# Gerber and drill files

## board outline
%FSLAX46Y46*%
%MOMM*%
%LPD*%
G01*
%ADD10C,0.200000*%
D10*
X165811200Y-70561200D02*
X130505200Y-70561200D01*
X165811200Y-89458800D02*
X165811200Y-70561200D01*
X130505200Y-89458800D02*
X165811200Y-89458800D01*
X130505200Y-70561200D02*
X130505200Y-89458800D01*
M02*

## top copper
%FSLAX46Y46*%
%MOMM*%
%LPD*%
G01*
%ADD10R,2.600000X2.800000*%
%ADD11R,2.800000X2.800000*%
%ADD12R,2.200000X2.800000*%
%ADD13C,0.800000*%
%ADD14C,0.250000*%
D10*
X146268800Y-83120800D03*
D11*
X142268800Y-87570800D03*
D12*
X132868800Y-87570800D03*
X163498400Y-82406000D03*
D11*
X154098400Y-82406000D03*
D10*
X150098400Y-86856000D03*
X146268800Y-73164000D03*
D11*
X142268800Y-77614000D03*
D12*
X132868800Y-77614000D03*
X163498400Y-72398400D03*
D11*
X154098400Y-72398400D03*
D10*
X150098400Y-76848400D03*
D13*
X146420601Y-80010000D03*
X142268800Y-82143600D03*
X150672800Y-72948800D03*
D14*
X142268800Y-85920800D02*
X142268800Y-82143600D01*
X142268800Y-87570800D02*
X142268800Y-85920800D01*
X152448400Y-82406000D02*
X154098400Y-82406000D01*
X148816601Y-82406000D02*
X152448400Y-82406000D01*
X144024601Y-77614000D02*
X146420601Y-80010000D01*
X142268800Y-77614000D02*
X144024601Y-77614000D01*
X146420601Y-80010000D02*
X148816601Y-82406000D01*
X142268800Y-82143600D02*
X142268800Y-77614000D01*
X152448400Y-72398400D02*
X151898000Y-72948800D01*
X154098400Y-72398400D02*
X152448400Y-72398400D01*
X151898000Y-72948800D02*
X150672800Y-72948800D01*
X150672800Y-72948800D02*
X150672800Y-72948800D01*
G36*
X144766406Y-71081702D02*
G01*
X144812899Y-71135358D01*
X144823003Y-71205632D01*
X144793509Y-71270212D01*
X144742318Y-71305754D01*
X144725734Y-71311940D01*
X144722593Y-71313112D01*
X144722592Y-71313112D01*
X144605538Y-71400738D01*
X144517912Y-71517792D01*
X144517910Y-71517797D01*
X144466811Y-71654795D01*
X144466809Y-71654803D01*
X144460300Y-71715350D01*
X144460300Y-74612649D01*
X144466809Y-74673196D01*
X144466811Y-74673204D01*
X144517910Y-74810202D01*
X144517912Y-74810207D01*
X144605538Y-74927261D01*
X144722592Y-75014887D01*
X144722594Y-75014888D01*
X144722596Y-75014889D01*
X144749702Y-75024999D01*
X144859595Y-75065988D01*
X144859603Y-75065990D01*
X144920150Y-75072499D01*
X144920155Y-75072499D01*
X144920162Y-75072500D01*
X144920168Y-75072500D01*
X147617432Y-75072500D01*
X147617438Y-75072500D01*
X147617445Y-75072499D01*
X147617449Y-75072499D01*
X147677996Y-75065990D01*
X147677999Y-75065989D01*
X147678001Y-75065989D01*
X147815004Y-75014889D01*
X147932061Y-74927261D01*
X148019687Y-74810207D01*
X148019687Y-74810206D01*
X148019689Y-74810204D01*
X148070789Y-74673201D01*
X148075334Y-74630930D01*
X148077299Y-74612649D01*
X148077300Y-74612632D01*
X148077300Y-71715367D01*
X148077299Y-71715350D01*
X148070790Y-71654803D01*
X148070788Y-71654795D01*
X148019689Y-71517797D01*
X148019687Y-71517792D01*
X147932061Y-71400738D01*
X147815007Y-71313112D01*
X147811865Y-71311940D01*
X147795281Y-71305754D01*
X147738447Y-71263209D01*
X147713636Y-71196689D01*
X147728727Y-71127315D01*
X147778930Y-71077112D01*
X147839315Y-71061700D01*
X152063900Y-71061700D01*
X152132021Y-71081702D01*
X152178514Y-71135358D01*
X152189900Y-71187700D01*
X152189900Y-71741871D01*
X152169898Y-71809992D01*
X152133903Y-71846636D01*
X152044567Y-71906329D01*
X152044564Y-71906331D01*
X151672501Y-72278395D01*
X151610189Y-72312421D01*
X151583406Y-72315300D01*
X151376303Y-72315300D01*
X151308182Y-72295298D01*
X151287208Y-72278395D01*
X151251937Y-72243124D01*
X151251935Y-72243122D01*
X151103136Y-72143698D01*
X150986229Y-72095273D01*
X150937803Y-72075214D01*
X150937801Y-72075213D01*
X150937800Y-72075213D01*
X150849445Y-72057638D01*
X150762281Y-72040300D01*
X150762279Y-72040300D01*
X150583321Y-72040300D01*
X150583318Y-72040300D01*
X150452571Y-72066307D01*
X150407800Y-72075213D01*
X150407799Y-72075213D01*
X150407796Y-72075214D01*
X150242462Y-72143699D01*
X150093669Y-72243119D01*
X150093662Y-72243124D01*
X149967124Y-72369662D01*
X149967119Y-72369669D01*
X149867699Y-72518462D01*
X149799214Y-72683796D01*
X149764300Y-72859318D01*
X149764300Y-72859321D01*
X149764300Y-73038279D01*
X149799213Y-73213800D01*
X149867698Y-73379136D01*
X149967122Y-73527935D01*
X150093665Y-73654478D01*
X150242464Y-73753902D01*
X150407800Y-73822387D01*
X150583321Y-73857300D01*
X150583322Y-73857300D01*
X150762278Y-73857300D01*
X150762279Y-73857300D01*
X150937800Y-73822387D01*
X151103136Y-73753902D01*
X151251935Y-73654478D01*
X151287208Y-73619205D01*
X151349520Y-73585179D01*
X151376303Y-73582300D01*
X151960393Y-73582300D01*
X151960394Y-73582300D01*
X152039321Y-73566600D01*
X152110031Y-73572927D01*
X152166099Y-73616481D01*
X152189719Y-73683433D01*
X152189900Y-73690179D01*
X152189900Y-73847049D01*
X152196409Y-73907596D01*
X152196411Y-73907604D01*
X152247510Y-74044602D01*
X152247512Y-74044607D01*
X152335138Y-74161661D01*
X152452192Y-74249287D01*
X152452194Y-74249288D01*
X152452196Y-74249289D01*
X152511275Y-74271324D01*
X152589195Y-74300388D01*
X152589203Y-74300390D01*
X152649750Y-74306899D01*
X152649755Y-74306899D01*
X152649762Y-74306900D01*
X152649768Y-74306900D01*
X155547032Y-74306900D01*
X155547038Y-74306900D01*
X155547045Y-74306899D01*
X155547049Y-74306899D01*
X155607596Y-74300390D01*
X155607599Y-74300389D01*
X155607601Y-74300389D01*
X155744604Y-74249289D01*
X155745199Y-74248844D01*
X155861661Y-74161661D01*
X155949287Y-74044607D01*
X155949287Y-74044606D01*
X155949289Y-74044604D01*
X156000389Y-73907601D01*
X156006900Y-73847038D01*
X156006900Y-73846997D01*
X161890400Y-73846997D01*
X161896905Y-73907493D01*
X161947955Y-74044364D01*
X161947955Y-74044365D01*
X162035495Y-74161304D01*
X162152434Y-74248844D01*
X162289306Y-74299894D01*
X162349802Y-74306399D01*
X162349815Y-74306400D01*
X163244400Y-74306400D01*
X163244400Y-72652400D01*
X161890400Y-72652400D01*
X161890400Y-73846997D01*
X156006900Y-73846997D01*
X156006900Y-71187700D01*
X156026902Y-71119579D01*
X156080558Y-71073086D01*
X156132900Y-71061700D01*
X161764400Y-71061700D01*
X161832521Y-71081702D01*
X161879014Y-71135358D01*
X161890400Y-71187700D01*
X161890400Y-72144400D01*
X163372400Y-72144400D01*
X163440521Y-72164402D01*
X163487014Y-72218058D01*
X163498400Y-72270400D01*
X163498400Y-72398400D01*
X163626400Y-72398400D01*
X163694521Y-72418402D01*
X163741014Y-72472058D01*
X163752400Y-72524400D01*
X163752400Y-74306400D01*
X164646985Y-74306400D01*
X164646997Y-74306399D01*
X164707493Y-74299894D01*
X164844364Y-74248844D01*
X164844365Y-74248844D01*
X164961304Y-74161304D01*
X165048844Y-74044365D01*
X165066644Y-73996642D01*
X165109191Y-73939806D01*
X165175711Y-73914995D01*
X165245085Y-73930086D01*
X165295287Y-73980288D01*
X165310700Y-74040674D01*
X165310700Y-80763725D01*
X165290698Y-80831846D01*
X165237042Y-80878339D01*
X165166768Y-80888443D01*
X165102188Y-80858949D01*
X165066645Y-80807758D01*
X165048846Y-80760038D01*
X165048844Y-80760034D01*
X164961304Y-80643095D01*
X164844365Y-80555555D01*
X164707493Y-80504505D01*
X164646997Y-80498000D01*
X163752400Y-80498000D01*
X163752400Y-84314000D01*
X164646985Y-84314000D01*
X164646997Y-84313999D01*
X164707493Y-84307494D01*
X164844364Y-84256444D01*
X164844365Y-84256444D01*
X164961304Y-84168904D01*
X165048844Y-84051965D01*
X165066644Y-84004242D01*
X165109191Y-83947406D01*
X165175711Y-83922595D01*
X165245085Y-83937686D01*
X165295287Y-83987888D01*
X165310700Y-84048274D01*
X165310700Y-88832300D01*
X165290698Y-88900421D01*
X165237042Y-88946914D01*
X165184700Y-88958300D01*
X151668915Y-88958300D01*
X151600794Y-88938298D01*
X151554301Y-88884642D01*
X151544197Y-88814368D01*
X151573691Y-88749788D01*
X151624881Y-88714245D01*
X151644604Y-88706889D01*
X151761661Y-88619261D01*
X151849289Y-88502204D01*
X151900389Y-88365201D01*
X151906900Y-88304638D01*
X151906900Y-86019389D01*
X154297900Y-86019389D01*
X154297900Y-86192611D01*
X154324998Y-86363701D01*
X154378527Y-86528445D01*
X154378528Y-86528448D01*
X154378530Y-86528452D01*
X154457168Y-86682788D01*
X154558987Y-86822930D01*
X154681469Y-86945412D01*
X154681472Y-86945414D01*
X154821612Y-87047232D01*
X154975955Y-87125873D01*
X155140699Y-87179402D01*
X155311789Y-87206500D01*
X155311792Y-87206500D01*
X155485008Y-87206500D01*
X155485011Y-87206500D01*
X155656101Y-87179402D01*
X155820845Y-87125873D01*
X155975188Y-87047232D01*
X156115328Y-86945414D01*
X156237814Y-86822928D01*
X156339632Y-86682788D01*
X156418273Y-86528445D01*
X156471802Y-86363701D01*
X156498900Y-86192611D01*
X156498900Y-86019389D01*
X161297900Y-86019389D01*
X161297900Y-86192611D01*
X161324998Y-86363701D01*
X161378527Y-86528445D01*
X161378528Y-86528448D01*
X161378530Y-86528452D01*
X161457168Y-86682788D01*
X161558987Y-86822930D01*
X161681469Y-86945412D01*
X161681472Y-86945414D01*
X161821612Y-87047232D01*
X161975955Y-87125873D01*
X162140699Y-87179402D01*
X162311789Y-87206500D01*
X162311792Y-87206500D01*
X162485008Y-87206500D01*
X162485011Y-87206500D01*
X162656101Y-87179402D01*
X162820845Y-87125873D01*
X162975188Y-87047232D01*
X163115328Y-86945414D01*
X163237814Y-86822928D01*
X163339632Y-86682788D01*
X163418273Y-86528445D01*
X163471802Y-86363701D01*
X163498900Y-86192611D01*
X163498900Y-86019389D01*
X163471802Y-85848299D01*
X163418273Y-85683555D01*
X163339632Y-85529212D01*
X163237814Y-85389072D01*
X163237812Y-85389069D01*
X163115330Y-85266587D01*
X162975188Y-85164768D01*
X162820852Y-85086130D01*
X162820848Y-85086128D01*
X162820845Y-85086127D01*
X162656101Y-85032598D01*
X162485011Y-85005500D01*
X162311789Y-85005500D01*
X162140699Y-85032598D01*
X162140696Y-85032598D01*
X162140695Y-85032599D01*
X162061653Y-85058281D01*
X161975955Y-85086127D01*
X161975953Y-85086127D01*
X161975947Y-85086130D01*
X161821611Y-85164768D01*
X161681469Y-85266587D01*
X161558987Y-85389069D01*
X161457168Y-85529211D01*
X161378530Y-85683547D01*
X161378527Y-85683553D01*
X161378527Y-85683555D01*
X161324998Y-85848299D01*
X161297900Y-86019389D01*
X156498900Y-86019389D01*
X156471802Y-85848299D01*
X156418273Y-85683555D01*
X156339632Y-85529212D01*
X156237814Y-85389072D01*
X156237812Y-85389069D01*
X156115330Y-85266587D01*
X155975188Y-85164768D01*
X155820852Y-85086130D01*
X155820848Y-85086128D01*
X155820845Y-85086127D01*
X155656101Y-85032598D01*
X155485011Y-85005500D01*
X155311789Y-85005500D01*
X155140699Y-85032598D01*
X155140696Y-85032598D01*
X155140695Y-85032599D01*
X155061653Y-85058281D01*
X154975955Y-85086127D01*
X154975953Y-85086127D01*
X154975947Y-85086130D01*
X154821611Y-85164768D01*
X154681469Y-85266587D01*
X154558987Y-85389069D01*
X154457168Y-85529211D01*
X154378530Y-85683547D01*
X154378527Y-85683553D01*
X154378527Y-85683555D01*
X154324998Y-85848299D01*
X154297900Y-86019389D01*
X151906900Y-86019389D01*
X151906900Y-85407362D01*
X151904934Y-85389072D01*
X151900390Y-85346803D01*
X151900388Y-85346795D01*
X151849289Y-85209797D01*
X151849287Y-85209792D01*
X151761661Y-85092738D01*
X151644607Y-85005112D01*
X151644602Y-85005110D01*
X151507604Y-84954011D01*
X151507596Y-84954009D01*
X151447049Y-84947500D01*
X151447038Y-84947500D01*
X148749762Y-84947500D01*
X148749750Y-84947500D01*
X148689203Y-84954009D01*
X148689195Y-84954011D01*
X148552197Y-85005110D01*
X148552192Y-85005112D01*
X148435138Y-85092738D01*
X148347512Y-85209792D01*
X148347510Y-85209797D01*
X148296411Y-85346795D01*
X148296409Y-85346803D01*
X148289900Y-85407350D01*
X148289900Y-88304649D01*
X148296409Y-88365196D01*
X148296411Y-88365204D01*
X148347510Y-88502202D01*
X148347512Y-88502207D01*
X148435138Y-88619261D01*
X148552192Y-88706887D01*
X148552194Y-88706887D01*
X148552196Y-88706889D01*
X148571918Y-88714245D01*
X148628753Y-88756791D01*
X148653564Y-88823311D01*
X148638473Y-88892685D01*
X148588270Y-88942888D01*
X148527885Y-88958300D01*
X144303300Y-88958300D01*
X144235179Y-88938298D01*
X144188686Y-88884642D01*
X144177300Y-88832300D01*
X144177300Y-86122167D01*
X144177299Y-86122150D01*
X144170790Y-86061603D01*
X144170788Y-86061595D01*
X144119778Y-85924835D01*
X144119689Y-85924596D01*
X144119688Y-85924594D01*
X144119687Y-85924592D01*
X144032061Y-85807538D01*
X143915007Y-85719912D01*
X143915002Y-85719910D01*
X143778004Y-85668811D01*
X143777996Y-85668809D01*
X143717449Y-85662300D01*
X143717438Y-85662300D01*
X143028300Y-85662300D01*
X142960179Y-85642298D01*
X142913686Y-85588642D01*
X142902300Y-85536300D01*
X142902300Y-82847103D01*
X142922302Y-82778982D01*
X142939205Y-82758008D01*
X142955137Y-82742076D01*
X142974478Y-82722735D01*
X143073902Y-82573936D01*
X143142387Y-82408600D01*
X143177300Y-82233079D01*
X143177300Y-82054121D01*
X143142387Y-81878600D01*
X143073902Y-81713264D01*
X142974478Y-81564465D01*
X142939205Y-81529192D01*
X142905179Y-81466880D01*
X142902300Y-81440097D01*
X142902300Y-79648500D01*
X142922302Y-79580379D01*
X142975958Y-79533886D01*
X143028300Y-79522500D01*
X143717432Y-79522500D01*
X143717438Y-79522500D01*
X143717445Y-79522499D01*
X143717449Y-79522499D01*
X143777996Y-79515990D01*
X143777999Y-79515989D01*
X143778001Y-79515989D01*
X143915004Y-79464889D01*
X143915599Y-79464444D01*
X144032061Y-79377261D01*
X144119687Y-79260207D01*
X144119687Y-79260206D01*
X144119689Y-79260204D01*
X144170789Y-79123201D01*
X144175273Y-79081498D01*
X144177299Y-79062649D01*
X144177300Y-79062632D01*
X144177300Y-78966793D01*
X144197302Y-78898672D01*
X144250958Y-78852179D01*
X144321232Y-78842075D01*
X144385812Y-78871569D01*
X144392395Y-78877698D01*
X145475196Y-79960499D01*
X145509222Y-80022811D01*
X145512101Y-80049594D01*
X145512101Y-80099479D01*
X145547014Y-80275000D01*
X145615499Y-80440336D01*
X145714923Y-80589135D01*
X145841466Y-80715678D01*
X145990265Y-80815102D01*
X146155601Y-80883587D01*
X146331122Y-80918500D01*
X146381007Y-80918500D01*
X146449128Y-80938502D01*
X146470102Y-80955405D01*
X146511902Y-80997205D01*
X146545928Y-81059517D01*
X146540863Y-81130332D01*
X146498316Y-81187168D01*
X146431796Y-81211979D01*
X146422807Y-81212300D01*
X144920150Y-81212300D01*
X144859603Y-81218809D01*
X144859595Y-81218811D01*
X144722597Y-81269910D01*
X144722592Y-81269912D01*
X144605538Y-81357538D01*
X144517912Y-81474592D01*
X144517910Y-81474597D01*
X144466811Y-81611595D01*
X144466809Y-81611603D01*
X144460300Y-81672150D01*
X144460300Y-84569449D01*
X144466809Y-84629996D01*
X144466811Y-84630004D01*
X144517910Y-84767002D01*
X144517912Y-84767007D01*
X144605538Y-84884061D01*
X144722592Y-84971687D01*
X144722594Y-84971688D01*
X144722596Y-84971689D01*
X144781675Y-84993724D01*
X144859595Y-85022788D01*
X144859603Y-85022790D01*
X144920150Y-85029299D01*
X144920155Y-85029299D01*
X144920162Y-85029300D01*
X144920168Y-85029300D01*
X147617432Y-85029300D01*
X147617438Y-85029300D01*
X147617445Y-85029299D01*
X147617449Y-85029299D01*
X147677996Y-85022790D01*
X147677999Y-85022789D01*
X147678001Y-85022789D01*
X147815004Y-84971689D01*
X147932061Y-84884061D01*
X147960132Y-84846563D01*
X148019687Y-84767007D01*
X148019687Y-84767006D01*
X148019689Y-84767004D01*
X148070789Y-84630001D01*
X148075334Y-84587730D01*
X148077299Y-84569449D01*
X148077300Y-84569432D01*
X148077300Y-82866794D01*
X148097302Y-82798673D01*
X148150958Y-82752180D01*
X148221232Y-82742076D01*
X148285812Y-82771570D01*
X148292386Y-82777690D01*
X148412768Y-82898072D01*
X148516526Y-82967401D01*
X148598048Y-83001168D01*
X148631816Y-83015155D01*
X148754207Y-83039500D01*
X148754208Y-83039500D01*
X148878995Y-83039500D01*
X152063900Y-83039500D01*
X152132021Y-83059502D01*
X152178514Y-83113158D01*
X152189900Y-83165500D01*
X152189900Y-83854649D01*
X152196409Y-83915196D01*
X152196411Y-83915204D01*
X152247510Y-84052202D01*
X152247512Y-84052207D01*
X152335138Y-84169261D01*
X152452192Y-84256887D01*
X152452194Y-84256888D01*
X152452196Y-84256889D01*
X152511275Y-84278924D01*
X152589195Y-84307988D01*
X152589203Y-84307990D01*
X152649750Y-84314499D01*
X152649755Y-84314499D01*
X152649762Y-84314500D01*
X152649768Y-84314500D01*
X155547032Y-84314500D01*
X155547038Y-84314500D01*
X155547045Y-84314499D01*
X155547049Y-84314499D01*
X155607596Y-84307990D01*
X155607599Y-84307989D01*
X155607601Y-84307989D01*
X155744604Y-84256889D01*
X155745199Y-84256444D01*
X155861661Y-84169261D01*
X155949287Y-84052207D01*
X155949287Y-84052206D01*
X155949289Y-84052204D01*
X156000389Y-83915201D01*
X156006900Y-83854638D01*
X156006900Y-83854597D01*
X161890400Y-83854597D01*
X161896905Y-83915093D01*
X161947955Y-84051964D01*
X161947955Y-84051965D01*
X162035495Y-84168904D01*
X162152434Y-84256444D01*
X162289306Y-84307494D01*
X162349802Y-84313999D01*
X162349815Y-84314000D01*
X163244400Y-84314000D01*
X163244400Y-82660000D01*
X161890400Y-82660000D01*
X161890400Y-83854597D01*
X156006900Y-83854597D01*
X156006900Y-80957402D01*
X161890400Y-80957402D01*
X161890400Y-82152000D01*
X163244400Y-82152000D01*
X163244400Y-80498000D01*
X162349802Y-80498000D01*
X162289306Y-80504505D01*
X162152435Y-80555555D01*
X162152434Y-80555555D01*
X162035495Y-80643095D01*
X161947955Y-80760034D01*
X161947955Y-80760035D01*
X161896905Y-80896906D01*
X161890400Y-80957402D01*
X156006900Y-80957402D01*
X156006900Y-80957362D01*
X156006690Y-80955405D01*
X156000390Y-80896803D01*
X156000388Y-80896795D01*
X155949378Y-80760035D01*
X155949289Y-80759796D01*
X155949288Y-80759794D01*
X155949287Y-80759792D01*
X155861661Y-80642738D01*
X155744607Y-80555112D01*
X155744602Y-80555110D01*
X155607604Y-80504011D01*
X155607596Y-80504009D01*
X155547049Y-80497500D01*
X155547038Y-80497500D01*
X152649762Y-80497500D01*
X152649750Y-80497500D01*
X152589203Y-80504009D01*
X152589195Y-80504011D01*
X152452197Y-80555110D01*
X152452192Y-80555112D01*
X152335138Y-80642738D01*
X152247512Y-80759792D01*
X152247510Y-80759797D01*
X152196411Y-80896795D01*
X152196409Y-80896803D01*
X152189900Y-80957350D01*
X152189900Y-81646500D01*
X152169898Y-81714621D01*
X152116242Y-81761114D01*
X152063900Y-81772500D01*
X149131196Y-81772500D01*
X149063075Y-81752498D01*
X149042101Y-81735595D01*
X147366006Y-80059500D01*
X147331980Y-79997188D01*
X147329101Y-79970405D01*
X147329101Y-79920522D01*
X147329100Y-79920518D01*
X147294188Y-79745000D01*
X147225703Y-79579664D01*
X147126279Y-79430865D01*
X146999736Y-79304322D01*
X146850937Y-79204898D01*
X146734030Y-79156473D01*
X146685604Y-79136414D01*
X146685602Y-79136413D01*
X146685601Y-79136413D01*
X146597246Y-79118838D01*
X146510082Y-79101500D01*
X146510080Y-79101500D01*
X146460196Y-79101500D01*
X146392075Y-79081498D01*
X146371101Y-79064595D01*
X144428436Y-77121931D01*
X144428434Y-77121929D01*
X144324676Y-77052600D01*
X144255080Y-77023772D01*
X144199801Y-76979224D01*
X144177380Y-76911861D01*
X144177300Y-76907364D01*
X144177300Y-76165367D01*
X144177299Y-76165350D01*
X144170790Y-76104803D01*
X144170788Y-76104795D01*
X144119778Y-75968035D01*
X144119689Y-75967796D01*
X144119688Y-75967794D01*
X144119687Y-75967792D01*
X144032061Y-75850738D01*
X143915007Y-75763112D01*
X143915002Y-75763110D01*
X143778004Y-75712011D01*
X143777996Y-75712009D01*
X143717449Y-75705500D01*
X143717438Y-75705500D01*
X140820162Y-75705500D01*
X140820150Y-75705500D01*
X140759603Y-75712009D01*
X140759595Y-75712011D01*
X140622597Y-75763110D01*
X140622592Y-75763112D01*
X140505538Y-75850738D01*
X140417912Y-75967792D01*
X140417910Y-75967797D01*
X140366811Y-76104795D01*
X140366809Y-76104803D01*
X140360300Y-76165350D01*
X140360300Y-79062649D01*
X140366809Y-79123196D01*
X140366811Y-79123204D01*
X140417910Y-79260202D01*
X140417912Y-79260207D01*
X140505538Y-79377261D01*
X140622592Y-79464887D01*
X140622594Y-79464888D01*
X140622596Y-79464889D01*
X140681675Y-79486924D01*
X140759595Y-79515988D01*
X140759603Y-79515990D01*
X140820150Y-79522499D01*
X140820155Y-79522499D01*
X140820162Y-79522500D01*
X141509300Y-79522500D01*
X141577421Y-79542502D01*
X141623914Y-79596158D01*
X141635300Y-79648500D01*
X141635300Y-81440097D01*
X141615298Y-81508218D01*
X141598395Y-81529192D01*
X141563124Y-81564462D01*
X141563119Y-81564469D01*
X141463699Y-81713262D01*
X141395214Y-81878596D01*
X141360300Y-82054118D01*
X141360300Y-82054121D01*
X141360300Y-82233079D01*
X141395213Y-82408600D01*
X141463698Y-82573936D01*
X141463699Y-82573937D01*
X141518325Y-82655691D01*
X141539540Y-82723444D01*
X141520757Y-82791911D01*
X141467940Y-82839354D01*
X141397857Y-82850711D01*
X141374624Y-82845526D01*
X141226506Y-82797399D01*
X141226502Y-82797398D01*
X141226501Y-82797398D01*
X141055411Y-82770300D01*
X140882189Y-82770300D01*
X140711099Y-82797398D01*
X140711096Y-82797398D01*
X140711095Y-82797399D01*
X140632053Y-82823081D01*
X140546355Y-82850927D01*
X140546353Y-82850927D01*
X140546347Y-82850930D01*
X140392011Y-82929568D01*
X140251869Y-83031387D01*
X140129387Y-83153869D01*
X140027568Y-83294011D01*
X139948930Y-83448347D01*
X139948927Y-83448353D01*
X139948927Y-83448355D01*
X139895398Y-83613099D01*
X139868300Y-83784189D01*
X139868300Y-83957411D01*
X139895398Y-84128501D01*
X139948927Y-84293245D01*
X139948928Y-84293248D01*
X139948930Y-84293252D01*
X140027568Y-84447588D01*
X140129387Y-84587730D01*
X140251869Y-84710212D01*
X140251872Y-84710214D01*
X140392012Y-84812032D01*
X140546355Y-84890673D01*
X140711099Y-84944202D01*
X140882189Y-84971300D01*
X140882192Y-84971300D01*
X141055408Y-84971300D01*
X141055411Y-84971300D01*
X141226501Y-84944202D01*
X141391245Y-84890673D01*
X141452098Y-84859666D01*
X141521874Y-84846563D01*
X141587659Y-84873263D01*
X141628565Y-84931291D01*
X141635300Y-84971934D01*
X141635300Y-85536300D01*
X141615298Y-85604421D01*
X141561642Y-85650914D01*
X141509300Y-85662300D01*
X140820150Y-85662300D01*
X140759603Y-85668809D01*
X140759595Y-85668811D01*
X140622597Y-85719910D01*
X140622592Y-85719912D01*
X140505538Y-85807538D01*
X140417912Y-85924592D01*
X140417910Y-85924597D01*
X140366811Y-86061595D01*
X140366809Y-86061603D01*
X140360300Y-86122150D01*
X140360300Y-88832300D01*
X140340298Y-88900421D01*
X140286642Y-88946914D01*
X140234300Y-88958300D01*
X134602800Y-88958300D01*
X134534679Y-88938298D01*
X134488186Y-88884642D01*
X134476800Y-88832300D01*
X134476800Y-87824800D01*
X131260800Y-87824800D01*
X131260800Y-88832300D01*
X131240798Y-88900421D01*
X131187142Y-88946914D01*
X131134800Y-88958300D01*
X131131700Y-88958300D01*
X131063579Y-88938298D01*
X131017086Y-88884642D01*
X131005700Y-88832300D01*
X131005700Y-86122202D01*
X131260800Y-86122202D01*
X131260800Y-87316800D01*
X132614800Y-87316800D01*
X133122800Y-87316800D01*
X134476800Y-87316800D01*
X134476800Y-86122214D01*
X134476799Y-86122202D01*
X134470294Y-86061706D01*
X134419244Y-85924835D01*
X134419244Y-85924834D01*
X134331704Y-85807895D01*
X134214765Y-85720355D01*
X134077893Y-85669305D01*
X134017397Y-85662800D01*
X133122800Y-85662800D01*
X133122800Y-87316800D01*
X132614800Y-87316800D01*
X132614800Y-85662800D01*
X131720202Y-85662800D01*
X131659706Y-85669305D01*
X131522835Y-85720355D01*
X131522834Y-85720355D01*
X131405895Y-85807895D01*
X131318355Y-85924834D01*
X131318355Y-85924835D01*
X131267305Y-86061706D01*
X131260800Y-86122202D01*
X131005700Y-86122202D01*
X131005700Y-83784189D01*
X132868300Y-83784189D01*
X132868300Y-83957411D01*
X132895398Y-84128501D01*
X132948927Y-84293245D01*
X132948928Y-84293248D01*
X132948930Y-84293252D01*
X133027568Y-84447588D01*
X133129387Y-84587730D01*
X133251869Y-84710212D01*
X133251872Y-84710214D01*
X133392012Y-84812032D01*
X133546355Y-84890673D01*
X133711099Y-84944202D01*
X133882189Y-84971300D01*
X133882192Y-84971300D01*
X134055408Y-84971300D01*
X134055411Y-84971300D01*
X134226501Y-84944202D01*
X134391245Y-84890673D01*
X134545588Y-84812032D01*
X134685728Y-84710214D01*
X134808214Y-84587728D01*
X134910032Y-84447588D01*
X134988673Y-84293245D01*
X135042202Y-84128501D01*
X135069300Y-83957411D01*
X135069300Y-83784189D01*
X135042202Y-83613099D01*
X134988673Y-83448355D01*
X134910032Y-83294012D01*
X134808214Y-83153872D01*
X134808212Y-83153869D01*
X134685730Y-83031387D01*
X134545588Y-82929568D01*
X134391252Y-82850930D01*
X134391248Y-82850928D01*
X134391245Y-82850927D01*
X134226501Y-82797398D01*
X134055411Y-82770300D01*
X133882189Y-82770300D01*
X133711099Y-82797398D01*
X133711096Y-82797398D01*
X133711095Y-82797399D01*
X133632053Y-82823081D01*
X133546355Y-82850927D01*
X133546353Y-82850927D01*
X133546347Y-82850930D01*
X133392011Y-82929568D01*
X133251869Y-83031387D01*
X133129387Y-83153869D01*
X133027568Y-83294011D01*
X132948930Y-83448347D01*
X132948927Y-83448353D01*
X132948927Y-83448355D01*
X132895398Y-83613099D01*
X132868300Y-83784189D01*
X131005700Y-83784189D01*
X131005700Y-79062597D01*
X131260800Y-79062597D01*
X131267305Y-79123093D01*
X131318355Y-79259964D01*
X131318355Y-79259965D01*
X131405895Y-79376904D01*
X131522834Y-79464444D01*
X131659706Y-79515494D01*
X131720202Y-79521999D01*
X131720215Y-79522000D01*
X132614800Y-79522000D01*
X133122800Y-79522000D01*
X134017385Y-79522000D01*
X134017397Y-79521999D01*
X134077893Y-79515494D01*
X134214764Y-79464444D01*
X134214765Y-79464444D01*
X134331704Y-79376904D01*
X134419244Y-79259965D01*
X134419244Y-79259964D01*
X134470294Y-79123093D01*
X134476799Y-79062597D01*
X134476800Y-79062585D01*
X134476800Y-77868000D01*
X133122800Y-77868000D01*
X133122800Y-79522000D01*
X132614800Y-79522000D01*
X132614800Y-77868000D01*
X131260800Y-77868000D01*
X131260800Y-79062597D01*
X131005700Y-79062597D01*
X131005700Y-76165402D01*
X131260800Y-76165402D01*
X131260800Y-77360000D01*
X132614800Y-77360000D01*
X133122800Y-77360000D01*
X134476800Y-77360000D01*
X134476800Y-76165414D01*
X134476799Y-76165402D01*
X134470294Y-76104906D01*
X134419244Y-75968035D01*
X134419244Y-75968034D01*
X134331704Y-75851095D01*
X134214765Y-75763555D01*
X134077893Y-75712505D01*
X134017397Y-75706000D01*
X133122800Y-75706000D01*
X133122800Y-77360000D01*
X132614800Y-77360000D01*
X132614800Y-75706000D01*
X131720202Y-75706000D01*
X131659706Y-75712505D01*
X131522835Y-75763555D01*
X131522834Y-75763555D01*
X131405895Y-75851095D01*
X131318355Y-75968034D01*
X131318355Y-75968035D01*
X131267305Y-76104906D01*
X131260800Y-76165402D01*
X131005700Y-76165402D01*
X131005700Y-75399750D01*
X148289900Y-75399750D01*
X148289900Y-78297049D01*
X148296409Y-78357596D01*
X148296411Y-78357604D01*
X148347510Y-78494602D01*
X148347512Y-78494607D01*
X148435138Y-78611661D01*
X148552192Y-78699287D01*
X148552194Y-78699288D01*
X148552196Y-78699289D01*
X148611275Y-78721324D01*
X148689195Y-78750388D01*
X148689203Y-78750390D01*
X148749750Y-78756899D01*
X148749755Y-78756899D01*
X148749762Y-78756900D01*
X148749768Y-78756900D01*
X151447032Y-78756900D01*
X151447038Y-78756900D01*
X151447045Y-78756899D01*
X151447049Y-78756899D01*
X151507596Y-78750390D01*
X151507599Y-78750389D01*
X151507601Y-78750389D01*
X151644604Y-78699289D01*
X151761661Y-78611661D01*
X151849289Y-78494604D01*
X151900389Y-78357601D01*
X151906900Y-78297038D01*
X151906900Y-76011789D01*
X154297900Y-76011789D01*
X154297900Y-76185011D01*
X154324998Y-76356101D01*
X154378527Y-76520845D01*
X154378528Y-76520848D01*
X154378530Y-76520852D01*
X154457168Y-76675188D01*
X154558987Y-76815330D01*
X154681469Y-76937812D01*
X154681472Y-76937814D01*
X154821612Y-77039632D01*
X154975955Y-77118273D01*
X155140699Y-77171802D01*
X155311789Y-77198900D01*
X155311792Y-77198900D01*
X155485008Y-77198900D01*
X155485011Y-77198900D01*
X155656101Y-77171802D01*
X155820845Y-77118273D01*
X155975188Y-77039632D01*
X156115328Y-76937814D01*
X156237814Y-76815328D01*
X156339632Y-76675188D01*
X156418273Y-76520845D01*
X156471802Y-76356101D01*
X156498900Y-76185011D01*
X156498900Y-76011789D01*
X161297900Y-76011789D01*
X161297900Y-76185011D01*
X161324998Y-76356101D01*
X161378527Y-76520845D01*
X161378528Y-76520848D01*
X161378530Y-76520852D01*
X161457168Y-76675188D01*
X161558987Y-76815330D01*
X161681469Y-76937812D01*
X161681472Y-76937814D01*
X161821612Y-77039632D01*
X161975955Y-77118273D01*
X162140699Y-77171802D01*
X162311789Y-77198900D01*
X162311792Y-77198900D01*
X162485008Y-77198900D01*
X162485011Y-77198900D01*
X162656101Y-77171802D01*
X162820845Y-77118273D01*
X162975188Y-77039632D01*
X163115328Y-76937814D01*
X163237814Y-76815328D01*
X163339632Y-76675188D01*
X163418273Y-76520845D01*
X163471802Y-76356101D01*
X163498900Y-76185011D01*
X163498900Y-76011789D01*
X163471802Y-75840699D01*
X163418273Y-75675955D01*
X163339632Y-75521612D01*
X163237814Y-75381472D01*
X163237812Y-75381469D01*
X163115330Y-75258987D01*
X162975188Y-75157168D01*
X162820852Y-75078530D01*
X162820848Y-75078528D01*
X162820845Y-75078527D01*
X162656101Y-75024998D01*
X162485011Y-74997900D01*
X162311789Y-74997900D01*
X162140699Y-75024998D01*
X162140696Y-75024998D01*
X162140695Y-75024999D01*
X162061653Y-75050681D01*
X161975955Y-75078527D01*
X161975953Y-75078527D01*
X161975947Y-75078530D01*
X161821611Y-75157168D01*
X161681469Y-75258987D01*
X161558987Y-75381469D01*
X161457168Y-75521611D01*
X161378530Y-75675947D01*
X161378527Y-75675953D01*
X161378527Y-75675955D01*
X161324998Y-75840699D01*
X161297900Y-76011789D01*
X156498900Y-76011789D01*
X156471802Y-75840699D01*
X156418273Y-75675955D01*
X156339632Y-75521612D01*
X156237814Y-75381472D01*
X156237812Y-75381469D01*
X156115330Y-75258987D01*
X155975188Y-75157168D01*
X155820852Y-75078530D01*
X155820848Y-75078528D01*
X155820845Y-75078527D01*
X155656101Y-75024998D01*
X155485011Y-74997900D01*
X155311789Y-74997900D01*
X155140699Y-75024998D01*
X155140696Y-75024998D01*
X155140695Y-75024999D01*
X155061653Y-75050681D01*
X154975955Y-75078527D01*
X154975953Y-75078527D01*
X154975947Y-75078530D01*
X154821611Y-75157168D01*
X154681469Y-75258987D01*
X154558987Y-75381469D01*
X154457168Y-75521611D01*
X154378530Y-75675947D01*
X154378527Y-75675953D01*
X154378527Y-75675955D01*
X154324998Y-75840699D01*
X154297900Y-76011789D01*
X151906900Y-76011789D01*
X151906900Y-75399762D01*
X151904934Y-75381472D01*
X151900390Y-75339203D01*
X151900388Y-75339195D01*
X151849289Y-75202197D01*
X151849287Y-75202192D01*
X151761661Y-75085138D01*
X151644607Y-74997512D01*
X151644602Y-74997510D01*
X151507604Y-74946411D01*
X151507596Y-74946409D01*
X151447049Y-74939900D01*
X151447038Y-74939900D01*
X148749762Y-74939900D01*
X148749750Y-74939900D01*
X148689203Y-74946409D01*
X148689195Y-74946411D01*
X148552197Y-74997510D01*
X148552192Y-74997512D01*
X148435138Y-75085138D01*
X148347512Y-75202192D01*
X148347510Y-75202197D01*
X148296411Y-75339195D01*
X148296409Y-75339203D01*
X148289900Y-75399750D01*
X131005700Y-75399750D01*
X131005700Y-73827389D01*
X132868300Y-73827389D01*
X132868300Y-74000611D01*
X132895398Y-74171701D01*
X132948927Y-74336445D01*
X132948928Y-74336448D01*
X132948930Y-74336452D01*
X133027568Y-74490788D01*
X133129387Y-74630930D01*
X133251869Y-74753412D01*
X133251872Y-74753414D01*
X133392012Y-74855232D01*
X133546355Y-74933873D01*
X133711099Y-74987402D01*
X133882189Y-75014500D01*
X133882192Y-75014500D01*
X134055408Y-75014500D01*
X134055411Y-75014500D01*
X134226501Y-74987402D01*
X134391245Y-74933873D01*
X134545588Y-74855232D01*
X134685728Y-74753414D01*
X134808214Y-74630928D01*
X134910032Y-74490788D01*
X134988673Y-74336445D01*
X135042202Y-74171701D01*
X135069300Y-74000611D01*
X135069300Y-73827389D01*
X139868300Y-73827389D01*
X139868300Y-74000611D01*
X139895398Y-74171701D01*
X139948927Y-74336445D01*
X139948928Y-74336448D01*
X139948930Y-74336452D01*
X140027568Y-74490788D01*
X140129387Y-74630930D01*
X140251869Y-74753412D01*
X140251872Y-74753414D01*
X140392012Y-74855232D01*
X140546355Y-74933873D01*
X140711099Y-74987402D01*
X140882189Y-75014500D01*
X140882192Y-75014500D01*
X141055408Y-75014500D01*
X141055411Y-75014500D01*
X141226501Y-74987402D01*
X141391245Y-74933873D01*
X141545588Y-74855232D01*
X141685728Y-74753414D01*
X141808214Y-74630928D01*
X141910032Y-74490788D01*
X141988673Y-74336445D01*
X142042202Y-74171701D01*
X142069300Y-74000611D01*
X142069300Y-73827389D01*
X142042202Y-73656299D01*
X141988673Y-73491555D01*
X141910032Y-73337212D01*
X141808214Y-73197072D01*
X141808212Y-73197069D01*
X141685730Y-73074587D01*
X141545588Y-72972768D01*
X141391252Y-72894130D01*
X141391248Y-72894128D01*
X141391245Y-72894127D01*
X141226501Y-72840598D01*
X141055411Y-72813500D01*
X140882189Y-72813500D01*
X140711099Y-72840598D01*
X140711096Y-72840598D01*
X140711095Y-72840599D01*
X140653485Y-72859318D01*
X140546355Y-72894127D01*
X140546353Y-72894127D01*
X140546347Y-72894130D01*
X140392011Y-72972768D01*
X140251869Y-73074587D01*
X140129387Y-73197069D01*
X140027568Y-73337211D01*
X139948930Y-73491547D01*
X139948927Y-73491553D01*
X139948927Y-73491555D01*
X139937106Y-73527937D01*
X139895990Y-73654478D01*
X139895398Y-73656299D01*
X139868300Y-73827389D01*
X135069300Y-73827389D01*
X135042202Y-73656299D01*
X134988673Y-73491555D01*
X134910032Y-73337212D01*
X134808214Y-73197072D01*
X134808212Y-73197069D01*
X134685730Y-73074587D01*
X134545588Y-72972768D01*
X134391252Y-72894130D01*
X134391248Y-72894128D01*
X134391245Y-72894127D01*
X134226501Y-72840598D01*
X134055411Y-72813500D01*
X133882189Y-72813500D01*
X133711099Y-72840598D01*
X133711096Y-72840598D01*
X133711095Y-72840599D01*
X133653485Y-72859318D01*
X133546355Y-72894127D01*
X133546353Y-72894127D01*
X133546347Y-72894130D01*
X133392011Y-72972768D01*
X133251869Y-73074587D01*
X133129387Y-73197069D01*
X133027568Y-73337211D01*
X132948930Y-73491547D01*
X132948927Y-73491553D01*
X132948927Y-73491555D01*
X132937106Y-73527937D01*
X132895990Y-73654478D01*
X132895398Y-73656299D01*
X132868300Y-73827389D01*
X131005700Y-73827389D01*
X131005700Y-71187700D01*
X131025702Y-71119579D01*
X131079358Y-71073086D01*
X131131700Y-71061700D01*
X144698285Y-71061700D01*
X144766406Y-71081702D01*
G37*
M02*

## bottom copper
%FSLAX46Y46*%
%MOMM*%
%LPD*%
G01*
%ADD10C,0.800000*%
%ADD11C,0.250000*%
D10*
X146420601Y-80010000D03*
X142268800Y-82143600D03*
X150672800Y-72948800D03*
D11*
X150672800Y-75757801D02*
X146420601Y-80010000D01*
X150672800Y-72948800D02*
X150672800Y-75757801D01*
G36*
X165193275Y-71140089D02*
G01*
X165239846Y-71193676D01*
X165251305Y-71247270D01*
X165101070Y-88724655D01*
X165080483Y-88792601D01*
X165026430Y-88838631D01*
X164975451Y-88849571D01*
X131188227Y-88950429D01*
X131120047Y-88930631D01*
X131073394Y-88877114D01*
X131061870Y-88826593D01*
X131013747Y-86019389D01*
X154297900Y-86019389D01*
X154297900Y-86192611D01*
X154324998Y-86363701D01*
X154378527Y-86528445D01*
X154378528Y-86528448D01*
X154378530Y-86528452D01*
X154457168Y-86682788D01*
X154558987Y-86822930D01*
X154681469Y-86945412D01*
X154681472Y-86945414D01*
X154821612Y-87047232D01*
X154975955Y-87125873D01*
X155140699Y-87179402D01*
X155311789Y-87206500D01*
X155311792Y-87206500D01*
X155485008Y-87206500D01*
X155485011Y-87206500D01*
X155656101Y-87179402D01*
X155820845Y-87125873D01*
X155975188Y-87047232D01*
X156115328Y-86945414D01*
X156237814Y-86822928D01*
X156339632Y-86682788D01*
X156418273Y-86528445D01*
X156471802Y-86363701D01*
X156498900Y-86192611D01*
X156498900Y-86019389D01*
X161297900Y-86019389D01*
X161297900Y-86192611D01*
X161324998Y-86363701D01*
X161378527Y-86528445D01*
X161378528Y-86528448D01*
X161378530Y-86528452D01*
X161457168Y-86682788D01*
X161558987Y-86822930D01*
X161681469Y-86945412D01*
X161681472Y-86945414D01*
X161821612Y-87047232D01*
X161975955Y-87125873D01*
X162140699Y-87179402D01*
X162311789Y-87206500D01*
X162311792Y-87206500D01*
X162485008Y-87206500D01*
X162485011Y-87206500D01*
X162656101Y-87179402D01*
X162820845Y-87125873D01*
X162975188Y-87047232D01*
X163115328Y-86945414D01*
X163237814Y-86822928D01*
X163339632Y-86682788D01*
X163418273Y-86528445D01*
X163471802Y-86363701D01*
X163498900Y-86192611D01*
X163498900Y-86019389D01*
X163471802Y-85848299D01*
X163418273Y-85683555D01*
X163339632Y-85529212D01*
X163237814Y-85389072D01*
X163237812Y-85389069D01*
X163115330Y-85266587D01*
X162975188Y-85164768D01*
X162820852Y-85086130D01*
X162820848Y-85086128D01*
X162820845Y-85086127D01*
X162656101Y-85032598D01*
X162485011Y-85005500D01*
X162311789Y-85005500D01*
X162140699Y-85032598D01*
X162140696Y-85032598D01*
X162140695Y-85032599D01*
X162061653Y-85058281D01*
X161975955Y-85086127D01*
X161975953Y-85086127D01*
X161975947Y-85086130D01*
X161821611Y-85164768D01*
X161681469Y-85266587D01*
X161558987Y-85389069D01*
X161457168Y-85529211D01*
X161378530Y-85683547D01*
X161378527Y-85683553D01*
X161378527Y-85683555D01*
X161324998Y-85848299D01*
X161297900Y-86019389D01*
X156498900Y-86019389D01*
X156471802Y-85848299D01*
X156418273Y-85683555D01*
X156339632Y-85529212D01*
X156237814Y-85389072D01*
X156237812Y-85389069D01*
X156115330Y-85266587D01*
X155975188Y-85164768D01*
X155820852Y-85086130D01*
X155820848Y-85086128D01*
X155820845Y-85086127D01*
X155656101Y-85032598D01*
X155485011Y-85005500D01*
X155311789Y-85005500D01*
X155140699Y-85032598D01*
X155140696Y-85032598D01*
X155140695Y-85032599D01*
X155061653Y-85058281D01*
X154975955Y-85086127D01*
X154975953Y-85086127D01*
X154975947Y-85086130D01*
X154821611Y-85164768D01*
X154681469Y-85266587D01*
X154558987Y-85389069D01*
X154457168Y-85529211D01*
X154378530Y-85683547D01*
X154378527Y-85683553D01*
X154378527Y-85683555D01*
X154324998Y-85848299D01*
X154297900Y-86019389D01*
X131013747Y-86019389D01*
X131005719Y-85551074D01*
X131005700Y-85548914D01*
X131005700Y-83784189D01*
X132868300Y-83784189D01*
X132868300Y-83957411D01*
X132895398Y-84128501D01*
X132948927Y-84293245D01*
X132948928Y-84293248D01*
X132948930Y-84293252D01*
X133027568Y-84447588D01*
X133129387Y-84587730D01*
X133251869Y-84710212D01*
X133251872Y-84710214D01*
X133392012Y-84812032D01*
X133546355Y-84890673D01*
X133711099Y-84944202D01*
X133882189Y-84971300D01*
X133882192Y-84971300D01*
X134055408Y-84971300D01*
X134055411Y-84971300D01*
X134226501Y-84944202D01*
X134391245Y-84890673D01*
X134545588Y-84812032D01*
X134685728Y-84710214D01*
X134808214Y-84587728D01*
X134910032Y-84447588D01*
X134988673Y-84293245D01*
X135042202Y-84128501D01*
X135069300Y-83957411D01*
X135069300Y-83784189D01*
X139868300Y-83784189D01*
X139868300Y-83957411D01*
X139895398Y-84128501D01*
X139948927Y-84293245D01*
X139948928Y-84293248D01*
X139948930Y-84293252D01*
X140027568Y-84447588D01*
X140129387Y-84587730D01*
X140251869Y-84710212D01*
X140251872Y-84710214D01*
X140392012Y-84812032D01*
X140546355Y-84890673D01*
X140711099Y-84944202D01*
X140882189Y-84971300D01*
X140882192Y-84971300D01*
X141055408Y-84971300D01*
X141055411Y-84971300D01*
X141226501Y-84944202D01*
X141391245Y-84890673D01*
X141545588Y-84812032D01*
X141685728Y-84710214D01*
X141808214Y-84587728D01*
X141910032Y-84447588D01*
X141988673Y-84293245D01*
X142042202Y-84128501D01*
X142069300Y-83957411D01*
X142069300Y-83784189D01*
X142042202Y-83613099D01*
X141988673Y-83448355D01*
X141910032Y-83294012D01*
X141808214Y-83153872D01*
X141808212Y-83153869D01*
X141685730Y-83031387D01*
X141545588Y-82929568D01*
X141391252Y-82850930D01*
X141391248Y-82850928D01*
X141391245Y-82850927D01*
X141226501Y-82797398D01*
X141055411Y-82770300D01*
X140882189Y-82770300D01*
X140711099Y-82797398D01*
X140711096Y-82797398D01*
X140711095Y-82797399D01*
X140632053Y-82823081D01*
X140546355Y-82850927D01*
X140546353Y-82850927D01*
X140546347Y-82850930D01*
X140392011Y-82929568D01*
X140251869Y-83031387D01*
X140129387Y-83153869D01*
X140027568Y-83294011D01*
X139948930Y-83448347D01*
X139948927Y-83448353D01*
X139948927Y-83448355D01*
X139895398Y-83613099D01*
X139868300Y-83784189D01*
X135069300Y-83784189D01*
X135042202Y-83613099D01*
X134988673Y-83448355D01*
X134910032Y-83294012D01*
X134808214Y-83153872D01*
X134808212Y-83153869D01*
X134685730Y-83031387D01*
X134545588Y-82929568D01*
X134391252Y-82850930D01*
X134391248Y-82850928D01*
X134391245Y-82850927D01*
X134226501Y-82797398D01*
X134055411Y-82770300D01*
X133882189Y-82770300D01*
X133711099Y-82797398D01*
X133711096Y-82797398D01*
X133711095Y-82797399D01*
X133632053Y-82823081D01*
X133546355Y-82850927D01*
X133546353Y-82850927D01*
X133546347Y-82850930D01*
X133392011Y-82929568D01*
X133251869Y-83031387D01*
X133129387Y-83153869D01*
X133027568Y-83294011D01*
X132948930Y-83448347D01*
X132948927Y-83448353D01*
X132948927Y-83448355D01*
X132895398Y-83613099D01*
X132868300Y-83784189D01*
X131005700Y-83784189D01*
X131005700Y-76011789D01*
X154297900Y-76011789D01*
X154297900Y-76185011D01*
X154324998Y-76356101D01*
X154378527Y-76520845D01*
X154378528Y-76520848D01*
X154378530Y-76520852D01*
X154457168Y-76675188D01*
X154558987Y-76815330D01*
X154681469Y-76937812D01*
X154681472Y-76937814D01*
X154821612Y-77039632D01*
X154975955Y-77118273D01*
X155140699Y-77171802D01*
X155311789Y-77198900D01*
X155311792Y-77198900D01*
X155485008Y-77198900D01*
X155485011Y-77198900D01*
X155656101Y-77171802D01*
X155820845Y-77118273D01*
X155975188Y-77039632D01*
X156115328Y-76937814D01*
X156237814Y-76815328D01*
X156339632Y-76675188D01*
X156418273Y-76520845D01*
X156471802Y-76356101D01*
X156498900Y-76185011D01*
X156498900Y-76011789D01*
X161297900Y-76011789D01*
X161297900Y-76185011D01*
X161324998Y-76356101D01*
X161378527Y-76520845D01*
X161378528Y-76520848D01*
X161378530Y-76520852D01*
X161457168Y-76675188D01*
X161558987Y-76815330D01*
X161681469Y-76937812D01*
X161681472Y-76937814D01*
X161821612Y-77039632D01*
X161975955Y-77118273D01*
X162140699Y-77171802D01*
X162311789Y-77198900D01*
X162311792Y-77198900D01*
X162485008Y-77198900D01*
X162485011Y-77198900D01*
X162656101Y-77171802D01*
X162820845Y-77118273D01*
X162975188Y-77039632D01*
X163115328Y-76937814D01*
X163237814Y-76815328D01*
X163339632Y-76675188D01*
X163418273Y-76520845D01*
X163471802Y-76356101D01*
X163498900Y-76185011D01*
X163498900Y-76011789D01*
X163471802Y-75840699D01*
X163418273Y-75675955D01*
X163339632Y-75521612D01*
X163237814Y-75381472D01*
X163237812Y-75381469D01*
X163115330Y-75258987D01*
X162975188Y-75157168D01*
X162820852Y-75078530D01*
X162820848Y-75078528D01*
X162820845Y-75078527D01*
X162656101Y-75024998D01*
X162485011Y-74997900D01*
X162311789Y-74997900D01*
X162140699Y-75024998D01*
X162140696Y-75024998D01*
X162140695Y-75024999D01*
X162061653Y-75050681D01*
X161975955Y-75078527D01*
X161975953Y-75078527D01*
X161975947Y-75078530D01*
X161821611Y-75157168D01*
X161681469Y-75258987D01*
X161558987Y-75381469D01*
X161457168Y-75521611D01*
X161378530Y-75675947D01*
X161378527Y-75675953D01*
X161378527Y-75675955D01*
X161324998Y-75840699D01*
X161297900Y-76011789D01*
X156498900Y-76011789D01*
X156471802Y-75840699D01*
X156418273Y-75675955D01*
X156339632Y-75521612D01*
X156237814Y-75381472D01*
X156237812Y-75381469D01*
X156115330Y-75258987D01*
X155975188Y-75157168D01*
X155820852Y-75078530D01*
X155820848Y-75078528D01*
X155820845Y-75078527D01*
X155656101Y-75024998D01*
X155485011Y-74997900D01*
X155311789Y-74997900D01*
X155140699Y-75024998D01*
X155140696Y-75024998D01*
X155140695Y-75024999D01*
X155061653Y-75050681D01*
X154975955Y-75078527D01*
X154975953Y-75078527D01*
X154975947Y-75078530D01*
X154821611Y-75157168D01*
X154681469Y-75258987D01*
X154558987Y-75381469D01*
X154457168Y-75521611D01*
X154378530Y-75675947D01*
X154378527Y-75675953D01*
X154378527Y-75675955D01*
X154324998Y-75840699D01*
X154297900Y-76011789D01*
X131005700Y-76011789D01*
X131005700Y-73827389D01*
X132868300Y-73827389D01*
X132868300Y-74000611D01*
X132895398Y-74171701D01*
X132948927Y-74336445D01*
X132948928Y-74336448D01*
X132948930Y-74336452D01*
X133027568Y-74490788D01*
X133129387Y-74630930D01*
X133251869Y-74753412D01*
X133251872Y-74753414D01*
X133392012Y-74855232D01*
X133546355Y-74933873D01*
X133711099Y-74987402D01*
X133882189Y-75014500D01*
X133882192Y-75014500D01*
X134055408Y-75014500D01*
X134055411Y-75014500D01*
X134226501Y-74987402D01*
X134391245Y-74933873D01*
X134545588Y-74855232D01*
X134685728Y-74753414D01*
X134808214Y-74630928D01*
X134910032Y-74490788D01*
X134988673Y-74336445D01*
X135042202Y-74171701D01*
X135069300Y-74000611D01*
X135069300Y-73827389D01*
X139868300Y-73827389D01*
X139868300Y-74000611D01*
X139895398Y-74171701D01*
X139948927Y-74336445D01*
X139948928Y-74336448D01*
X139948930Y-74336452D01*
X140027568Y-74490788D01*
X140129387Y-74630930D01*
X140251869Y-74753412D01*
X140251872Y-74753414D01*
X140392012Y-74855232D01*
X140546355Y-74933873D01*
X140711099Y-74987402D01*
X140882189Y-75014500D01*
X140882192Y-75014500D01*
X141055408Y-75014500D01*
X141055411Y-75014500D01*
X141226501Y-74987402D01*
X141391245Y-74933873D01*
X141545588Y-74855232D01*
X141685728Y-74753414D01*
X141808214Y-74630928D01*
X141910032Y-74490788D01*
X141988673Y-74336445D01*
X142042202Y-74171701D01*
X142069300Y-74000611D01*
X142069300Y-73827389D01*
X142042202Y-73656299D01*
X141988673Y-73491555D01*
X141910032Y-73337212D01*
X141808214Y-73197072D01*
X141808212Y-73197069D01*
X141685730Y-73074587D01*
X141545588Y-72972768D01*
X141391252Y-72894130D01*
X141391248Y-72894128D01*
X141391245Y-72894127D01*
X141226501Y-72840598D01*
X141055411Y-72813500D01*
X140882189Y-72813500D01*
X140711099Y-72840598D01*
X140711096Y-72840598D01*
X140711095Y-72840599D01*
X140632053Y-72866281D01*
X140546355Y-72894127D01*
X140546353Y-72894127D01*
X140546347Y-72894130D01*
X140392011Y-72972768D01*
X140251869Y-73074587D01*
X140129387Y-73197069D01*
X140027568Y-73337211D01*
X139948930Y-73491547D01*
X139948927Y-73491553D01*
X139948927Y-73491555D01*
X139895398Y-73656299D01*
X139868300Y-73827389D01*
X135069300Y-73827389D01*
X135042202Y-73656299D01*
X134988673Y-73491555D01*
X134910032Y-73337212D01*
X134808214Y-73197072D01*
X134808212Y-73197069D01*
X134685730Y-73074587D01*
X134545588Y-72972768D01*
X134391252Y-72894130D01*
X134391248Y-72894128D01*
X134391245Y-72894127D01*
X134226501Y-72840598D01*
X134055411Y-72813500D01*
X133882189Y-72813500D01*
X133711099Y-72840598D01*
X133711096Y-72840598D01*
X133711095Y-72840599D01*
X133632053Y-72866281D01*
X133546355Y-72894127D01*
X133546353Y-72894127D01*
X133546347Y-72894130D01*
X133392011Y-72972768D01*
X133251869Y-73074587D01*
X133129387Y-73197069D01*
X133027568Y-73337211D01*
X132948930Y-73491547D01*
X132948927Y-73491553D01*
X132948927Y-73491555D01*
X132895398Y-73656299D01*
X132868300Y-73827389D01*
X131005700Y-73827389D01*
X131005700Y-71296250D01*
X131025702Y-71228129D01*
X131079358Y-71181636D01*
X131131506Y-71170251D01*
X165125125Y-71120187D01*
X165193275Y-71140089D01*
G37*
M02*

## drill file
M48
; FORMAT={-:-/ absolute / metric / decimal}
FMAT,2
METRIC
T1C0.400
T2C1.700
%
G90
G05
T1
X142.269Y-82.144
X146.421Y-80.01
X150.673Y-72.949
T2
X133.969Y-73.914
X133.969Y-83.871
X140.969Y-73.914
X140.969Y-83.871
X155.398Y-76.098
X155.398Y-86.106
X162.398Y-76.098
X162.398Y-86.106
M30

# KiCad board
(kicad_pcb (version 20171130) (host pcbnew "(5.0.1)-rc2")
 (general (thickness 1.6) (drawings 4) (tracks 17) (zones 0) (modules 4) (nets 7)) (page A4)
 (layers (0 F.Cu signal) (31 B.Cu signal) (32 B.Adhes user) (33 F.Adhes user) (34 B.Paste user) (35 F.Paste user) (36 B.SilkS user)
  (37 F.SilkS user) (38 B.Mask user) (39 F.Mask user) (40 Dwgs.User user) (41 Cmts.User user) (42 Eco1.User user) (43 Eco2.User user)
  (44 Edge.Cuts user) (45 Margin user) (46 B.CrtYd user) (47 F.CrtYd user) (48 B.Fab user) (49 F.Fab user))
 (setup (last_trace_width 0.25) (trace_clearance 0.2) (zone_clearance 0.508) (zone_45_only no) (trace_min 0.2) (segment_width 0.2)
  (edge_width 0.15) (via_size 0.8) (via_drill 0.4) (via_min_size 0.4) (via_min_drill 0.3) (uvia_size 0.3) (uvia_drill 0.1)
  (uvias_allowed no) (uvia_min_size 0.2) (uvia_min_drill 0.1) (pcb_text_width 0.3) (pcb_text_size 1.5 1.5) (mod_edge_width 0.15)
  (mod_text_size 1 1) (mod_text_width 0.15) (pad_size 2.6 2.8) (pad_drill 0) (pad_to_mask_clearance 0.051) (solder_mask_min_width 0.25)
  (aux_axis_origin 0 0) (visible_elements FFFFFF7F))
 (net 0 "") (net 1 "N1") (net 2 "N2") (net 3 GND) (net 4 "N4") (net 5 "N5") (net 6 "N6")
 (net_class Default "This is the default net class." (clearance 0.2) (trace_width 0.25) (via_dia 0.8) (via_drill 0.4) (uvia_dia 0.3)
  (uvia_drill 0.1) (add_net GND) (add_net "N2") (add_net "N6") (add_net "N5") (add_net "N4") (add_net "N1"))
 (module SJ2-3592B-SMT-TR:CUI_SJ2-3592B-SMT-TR (layer F.Cu) (at 137.7188 83.8708)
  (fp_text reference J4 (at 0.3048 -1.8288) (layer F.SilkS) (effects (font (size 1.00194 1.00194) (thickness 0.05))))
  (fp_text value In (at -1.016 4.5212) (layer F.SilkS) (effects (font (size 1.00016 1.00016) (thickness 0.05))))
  (pad Hole np_thru_hole circle (at 3.25 0) (size 1.7 1.7) (drill 1.7) (layers *.Cu *.Mask F.SilkS))
  (pad Hole np_thru_hole circle (at -3.75 0) (size 1.7 1.7) (drill 1.7) (layers *.Cu *.Mask F.SilkS))
  (pad TN smd rect (at 8.55 -0.75) (size 2.6 2.8) (layers F.Cu F.Paste F.Mask) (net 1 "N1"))
  (pad T smd rect (at 4.55 3.7) (size 2.8 2.8) (layers F.Cu F.Paste F.Mask) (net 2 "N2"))
  (pad S smd rect (at -4.85 3.7) (size 2.2 2.8) (layers F.Cu F.Paste F.Mask) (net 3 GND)))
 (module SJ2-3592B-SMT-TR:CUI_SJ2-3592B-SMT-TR (layer F.Cu) (at 158.6484 86.106 180)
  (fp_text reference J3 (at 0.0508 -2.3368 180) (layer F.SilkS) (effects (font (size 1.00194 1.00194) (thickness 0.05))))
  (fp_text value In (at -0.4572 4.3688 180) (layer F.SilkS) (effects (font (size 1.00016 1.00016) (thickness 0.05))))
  (pad S smd rect (at -4.85 3.7 180) (size 2.2 2.8) (layers F.Cu F.Paste F.Mask) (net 3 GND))
  (pad T smd rect (at 4.55 3.7 180) (size 2.8 2.8) (layers F.Cu F.Paste F.Mask) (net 2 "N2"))
  (pad TN smd rect (at 8.55 -0.75 180) (size 2.6 2.8) (layers F.Cu F.Paste F.Mask) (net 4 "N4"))
  (pad Hole np_thru_hole circle (at -3.75 0 180) (size 1.7 1.7) (drill 1.7) (layers *.Cu *.Mask F.SilkS))
  (pad Hole np_thru_hole circle (at 3.25 0 180) (size 1.7 1.7) (drill 1.7) (layers *.Cu *.Mask F.SilkS)))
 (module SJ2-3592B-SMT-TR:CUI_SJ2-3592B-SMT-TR (layer F.Cu) (at 137.7188 73.914)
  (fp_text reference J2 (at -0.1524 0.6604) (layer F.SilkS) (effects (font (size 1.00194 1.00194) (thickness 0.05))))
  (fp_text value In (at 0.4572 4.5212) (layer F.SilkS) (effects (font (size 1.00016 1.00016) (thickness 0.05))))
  (pad Hole np_thru_hole circle (at 3.25 0) (size 1.7 1.7) (drill 1.7) (layers *.Cu *.Mask F.SilkS))
  (pad Hole np_thru_hole circle (at -3.75 0) (size 1.7 1.7) (drill 1.7) (layers *.Cu *.Mask F.SilkS))
  (pad TN smd rect (at 8.55 -0.75) (size 2.6 2.8) (layers F.Cu F.Paste F.Mask) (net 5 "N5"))
  (pad T smd rect (at 4.55 3.7) (size 2.8 2.8) (layers F.Cu F.Paste F.Mask) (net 2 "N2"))
  (pad S smd rect (at -4.85 3.7) (size 2.2 2.8) (layers F.Cu F.Paste F.Mask) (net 3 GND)))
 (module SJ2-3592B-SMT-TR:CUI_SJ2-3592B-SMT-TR (layer F.Cu) (at 158.6484 76.0984 180)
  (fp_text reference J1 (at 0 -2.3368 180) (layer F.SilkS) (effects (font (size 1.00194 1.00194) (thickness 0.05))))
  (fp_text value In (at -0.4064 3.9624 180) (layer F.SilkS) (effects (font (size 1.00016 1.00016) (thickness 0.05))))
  (pad S smd rect (at -4.85 3.7 180) (size 2.2 2.8) (layers F.Cu F.Paste F.Mask) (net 3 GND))
  (pad T smd rect (at 4.55 3.7 180) (size 2.8 2.8) (layers F.Cu F.Paste F.Mask) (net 2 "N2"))
  (pad TN smd rect (at 8.55 -0.75 180) (size 2.6 2.8) (layers F.Cu F.Paste F.Mask) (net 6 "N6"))
  (pad Hole np_thru_hole circle (at -3.75 0 180) (size 1.7 1.7) (drill 1.7) (layers *.Cu *.Mask F.SilkS))
  (pad Hole np_thru_hole circle (at 3.25 0 180) (size 1.7 1.7) (drill 1.7) (layers *.Cu *.Mask F.SilkS)))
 (gr_line (start 165.8112 70.5612) (end 130.5052 70.5612) (layer Edge.Cuts) (width 0.2))
 (gr_line (start 165.8112 89.4588) (end 165.8112 70.5612) (layer Edge.Cuts) (width 0.2))
 (gr_line (start 130.5052 89.4588) (end 165.8112 89.4588) (layer Edge.Cuts) (width 0.2))
 (gr_line (start 130.5052 70.5612) (end 130.5052 89.4588) (layer Edge.Cuts) (width 0.2))
 (segment (start 142.2688 85.9208) (end 142.2688 82.1436) (width 0.25) (layer F.Cu) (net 2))
 (segment (start 142.2688 87.5708) (end 142.2688 85.9208) (width 0.25) (layer F.Cu) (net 2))
 (segment (start 152.4484 82.406) (end 154.0984 82.406) (width 0.25) (layer F.Cu) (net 2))
 (segment (start 148.816601 82.406) (end 152.4484 82.406) (width 0.25) (layer F.Cu) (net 2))
 (segment (start 144.024601 77.614) (end 146.420601 80.01) (width 0.25) (layer F.Cu) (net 2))
 (segment (start 142.2688 77.614) (end 144.024601 77.614) (width 0.25) (layer F.Cu) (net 2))
 (segment (start 146.420601 80.01) (end 148.816601 82.406) (width 0.25) (layer F.Cu) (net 2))
 (via (at 146.420601 80.01) (size 0.8) (drill 0.4) (layers F.Cu B.Cu) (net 2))
 (segment (start 142.2688 82.1436) (end 142.2688 77.614) (width 0.25) (layer F.Cu) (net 2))
 (via (at 142.2688 82.1436) (size 0.8) (drill 0.4) (layers F.Cu B.Cu) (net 2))
 (segment (start 152.4484 72.3984) (end 151.898 72.9488) (width 0.25) (layer F.Cu) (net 2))
 (segment (start 154.0984 72.3984) (end 152.4484 72.3984) (width 0.25) (layer F.Cu) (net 2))
 (segment (start 151.898 72.9488) (end 150.6728 72.9488) (width 0.25) (layer F.Cu) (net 2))
 (segment (start 150.6728 72.9488) (end 150.6728 72.9488) (width 0.25) (layer F.Cu) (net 2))
 (via (at 150.6728 72.9488) (size 0.8) (drill 0.4) (layers F.Cu B.Cu) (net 2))
 (segment (start 150.6728 75.757801) (end 146.420601 80.01) (width 0.25) (layer B.Cu) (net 2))
 (segment (start 150.6728 72.9488) (end 150.6728 75.757801) (width 0.25) (layer B.Cu) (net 2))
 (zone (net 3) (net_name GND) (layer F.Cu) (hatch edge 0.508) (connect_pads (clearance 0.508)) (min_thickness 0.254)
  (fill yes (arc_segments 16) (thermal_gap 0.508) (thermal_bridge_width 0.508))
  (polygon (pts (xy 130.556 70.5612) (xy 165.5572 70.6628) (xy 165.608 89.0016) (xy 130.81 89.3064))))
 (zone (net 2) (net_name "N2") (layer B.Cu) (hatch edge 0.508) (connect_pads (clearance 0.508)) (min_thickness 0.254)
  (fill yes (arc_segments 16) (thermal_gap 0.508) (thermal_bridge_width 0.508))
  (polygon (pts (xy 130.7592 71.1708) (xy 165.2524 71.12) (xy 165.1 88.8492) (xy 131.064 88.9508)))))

